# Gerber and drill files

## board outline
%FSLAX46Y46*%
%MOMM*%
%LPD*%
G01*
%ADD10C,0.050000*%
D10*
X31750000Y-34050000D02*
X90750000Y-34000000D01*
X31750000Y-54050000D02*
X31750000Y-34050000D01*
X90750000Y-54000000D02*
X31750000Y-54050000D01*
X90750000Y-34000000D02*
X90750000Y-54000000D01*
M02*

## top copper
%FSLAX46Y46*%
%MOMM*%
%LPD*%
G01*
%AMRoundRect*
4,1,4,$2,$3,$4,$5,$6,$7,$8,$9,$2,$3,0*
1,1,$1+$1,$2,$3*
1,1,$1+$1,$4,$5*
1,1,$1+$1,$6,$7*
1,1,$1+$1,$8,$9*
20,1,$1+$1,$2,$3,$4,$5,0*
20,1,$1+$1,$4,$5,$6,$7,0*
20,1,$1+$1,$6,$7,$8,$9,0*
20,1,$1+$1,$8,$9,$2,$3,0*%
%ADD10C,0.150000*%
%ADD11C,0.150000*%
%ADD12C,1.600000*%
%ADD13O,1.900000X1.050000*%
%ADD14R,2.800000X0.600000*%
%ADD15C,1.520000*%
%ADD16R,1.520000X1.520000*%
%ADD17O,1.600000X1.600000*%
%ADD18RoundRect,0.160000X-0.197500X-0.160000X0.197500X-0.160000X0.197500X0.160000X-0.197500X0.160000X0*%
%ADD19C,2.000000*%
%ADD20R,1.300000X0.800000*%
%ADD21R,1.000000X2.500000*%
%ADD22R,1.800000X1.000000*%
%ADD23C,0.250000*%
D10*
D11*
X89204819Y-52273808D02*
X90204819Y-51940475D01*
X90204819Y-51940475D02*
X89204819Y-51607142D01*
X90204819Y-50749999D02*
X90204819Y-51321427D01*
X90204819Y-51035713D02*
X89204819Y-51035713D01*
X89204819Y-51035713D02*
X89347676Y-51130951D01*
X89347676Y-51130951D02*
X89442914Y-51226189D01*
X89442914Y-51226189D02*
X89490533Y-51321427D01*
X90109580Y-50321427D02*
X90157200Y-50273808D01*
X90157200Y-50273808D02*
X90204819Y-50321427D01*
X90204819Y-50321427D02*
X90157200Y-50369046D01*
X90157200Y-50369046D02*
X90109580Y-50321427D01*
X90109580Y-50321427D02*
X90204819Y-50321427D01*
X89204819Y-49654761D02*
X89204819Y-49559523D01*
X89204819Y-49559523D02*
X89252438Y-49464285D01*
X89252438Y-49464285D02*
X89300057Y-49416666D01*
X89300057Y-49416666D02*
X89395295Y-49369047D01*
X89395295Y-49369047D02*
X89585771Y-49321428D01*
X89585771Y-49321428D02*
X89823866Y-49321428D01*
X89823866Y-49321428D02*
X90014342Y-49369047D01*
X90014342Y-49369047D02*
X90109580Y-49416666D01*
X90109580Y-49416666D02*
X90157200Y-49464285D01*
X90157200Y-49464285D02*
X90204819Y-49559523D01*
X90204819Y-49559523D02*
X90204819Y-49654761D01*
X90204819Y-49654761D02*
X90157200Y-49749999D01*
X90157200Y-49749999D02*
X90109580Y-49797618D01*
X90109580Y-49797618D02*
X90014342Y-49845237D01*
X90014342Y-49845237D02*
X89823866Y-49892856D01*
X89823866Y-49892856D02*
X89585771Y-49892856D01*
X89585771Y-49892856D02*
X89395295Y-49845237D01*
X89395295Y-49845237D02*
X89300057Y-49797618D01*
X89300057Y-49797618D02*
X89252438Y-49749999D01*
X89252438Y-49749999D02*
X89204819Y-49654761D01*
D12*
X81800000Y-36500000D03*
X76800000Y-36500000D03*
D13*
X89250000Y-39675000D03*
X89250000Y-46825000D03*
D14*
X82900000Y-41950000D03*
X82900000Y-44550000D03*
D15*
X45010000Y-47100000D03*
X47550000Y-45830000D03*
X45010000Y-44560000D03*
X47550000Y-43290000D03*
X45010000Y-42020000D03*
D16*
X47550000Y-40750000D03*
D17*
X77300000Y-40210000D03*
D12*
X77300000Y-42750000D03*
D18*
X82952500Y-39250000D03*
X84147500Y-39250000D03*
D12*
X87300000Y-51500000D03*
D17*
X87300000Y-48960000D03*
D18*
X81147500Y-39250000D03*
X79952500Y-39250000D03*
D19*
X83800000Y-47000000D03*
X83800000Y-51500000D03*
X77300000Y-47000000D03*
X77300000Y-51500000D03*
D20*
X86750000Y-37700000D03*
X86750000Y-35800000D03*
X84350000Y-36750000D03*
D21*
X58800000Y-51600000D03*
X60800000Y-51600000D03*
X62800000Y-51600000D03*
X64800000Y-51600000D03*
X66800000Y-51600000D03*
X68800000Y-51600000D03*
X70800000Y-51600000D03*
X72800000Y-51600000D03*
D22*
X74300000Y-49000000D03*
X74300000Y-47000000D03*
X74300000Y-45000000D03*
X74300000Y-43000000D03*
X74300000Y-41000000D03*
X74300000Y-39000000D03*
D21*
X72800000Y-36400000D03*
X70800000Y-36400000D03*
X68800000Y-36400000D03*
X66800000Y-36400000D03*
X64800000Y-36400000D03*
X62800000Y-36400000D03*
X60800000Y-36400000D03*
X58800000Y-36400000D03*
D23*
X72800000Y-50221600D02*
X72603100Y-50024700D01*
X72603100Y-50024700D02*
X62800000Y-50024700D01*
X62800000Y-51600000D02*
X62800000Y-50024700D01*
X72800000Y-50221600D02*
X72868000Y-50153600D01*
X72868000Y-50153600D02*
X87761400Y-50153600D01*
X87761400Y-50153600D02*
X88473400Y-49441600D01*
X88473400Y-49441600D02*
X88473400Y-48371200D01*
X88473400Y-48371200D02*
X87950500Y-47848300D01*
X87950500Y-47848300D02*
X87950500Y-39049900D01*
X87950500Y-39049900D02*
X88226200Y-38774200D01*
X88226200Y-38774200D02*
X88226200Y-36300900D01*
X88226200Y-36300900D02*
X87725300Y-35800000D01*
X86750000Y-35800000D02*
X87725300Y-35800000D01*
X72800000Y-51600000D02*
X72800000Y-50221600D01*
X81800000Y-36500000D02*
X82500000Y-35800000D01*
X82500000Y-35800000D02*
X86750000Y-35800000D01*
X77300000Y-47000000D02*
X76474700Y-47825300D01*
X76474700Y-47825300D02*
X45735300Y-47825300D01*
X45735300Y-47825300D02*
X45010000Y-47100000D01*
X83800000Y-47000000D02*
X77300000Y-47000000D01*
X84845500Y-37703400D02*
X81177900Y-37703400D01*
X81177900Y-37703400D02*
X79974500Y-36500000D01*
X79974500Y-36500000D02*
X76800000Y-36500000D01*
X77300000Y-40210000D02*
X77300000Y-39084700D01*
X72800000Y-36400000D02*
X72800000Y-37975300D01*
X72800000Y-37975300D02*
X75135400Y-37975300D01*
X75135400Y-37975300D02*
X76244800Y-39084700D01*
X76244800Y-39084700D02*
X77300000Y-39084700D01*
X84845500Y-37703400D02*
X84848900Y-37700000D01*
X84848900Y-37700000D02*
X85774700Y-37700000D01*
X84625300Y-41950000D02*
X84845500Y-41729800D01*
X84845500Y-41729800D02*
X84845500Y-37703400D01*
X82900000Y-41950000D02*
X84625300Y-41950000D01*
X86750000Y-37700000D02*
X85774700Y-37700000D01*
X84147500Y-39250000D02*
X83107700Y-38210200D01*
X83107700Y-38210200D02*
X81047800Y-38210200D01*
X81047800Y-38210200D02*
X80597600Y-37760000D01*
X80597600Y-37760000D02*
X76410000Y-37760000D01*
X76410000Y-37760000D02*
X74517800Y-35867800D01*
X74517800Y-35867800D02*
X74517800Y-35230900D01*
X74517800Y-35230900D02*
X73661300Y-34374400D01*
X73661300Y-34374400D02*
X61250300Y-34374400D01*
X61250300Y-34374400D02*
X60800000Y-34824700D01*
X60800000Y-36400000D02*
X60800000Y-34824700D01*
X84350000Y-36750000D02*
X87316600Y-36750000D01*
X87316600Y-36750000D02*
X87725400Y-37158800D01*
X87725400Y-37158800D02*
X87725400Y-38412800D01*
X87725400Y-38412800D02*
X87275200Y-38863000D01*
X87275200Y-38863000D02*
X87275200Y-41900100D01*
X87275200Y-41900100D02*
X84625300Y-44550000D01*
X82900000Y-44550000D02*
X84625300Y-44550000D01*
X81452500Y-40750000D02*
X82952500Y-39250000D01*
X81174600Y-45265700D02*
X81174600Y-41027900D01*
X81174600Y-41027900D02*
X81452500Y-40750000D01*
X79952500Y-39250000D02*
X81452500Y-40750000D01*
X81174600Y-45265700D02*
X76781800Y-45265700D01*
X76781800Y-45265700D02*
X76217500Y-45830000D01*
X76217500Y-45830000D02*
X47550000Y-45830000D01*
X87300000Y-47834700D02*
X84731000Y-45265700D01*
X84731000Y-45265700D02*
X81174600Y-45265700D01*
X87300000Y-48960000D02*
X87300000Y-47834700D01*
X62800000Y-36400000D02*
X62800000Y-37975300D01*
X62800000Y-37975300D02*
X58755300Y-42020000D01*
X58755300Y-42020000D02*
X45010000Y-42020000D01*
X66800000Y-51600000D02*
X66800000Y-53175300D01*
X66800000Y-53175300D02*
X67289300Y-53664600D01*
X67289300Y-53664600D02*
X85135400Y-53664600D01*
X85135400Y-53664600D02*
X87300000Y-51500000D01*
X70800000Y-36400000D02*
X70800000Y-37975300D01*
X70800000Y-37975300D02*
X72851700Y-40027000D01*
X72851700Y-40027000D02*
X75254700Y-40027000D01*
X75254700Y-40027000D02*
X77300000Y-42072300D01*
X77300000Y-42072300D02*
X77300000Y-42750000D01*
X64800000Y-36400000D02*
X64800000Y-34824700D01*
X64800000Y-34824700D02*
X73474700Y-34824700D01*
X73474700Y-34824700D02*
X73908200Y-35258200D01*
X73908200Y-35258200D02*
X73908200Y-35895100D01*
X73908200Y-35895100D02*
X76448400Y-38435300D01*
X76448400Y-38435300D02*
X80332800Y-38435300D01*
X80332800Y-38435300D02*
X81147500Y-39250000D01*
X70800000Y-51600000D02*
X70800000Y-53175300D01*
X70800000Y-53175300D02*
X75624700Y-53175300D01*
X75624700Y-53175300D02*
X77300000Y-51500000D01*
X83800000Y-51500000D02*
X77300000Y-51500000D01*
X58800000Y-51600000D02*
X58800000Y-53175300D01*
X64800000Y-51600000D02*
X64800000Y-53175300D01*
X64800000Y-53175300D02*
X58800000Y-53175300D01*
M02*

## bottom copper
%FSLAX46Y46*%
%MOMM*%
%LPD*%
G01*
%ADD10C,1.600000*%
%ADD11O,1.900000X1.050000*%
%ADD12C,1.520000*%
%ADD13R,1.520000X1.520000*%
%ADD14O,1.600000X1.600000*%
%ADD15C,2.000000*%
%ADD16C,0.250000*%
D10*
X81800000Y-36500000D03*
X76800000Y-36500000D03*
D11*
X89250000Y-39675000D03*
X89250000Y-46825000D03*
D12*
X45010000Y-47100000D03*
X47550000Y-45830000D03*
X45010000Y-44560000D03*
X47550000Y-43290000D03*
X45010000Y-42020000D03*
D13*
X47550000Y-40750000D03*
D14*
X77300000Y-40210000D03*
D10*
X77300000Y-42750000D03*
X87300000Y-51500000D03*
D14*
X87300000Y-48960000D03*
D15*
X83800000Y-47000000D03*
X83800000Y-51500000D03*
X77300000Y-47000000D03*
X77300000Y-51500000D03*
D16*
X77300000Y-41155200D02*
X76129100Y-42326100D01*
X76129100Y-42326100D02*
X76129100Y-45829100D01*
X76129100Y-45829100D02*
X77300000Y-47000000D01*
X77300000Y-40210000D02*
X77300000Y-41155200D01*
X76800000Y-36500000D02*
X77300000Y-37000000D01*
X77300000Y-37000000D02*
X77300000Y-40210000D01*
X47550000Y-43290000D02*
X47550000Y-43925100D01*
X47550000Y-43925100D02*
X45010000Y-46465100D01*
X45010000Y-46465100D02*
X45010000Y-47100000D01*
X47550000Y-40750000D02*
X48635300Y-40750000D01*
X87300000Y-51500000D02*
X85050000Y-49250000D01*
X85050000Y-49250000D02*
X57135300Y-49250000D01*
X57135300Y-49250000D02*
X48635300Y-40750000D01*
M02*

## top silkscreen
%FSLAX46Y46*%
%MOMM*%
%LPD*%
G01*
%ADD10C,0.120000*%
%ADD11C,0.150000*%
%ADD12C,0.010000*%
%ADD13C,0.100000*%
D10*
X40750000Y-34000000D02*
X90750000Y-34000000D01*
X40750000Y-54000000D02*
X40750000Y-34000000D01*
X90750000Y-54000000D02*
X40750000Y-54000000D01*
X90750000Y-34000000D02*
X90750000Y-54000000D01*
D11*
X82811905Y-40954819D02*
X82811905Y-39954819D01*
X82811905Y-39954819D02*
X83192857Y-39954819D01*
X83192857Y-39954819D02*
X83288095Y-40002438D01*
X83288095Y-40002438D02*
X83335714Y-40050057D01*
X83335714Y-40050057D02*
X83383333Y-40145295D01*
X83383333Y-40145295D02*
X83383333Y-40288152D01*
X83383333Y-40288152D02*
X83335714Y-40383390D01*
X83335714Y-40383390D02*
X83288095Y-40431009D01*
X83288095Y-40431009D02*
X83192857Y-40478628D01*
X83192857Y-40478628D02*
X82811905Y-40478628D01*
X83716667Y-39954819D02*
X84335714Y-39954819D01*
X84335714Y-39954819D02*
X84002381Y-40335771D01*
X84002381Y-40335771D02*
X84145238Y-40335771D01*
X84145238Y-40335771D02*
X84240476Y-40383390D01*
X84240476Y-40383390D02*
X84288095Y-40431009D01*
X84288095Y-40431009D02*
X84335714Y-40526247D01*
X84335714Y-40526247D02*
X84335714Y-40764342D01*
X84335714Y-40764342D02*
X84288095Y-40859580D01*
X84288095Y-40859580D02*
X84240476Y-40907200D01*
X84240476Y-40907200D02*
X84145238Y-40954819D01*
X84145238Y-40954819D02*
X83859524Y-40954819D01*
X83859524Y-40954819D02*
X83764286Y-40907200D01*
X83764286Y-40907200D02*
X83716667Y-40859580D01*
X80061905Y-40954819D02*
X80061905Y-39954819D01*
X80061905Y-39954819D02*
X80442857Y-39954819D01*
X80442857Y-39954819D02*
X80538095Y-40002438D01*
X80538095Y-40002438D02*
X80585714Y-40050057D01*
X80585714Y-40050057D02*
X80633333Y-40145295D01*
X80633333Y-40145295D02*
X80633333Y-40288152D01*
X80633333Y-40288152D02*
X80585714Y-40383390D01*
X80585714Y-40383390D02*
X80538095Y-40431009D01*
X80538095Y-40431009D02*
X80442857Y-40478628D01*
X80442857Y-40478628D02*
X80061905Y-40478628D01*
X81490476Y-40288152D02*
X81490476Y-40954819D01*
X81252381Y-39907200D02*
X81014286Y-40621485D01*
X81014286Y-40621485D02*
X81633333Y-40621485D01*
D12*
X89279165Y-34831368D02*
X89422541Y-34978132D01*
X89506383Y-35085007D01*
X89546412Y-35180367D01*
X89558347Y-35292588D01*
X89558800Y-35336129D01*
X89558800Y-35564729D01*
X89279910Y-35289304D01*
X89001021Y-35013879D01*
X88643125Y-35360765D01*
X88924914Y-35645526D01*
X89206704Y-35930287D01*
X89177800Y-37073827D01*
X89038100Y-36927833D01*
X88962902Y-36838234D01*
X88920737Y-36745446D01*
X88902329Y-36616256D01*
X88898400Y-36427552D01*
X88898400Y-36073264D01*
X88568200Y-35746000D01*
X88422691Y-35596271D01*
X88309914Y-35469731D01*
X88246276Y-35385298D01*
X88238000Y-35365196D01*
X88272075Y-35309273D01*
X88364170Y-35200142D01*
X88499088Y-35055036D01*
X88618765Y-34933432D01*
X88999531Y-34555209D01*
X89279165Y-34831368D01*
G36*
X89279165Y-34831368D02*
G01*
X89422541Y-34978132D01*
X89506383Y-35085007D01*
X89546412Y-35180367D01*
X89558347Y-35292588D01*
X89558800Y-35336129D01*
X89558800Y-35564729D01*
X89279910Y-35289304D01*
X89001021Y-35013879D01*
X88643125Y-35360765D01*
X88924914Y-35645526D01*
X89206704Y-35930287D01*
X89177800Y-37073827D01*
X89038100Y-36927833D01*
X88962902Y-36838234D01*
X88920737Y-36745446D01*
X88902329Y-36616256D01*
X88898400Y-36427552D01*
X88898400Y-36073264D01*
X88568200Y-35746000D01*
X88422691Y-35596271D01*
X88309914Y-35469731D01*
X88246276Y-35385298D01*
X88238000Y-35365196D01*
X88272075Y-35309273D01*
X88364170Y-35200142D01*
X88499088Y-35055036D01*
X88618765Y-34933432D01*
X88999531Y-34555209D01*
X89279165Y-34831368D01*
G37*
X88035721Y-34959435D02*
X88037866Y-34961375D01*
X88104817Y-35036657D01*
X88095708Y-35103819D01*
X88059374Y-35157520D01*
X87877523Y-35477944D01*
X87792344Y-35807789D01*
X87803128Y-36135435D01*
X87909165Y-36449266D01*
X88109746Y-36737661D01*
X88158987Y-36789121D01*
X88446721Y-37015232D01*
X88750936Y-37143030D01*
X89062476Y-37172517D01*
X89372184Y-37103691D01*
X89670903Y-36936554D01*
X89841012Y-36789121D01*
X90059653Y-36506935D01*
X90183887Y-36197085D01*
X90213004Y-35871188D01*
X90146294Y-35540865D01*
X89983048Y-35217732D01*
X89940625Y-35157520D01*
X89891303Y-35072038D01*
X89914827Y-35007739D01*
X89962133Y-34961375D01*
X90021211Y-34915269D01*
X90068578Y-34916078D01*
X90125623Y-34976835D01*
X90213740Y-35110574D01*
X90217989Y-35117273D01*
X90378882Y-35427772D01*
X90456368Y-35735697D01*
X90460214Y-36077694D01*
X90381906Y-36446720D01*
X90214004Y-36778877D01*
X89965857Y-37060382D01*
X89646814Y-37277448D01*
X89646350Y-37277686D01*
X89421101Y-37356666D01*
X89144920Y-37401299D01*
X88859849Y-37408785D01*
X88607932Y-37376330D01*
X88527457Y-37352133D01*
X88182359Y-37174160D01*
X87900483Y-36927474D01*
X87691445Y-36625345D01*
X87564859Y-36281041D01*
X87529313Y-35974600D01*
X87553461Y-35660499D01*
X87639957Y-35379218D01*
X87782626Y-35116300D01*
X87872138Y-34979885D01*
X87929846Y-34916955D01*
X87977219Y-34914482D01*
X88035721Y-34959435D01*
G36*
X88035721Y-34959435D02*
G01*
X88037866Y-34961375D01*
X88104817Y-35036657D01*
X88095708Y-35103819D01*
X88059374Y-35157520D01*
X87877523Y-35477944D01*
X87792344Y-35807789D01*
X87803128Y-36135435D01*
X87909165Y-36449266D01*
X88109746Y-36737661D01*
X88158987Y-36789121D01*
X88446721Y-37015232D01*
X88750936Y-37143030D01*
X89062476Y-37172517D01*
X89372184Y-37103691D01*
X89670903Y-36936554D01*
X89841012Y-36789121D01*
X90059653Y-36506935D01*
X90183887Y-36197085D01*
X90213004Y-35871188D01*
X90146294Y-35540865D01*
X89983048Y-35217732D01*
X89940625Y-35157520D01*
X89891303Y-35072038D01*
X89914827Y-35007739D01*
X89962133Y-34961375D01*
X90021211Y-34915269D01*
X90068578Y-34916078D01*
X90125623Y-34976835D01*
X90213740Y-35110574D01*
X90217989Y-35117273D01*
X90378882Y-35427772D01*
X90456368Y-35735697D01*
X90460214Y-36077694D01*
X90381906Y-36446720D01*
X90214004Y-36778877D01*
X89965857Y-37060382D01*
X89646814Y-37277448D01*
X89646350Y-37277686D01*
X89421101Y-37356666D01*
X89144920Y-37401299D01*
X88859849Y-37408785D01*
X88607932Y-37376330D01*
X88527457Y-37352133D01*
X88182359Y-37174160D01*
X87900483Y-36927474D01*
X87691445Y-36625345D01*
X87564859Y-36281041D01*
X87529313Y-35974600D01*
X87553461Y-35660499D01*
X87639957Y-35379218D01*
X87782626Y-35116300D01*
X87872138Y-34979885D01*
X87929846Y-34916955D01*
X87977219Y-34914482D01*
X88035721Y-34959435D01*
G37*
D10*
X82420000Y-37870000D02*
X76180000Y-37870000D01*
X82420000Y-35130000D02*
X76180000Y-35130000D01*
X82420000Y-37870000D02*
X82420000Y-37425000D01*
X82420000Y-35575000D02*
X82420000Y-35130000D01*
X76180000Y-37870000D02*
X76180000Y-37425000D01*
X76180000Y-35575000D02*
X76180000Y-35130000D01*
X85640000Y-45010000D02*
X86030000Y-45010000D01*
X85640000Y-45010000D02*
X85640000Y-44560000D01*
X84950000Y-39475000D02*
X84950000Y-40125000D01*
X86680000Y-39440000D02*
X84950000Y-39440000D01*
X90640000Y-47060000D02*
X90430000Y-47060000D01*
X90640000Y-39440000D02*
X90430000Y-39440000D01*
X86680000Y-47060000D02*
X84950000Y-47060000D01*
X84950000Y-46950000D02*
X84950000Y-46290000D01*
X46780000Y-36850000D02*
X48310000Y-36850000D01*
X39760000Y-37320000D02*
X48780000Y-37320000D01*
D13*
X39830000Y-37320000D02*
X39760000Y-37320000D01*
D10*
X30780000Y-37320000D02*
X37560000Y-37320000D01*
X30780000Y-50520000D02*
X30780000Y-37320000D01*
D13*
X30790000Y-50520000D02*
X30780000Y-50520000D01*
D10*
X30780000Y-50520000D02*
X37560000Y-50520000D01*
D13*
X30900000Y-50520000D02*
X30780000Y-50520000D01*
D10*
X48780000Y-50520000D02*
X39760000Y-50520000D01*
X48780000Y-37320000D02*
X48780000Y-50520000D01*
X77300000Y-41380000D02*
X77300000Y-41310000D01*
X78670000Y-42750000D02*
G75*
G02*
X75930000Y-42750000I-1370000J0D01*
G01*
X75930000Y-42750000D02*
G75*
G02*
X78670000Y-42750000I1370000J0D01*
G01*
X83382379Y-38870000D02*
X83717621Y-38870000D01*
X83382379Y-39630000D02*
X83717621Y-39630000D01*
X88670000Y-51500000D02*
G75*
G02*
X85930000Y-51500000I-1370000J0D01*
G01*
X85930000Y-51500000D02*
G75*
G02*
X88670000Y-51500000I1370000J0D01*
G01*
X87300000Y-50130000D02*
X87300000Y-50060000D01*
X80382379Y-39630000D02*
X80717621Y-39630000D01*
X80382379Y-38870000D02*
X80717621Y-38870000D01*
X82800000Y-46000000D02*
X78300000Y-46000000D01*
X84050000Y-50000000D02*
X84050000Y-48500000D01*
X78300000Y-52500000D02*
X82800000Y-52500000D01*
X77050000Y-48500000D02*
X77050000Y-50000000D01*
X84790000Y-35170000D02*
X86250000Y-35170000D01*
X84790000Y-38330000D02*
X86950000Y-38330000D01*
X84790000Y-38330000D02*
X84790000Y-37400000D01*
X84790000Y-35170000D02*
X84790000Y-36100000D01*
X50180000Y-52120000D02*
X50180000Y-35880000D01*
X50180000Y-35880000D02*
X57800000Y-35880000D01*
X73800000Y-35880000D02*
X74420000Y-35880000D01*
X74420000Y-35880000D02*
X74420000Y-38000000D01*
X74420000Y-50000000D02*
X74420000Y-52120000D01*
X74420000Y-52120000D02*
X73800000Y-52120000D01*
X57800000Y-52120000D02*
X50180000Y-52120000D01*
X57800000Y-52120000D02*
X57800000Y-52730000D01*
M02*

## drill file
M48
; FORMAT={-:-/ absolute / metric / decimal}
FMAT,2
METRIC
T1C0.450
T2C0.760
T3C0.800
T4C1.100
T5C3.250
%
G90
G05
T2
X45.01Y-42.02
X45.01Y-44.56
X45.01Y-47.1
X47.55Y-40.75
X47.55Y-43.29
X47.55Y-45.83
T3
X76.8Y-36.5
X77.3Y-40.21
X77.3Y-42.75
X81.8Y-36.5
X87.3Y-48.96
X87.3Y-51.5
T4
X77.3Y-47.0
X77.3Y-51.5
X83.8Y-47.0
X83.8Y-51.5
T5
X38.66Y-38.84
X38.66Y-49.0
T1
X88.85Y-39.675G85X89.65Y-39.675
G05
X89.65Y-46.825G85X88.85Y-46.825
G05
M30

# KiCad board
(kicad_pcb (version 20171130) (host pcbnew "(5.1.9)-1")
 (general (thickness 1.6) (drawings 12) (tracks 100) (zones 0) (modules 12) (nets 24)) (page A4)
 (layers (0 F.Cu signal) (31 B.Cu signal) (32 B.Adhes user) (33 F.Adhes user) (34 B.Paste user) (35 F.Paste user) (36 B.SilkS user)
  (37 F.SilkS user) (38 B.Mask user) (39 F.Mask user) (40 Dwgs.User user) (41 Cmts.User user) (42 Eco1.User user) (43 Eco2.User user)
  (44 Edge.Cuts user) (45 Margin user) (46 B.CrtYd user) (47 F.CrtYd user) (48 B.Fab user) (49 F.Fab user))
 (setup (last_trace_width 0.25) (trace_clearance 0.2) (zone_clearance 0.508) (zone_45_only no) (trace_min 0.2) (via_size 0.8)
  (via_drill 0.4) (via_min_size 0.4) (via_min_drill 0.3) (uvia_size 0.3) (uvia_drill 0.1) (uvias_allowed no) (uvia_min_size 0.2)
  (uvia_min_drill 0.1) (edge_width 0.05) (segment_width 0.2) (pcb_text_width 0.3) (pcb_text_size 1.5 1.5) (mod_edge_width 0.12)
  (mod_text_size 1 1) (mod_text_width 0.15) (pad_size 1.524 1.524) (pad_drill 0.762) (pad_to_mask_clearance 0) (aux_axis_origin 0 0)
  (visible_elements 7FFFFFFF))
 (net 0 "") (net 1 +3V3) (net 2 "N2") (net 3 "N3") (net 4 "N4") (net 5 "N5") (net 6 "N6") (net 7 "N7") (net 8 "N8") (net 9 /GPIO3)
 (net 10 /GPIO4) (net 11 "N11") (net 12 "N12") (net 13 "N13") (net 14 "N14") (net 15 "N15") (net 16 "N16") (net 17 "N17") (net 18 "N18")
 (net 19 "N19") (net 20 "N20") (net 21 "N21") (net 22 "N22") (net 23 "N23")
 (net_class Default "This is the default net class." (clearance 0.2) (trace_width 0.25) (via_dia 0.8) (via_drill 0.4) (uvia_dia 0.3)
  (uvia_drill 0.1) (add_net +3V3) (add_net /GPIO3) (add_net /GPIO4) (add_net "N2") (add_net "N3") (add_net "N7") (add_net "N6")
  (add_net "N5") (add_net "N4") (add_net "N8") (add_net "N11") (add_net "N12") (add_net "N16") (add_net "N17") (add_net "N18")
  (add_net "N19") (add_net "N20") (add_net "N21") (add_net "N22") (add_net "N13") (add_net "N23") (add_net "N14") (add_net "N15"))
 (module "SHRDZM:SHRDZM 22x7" (layer B.Cu) (at 63 43.25 180)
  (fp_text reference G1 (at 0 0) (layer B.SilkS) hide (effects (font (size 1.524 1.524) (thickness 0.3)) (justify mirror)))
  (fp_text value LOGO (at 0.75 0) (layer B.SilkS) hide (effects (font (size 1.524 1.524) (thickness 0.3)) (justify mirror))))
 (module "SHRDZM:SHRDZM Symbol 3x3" (layer F.Cu) (at 89 36)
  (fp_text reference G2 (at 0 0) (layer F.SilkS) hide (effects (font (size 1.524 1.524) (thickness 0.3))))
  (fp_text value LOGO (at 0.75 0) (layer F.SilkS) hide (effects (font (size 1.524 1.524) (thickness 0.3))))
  (fp_poly
   (pts (xy 0.279165 -1.168632) (xy 0.422541 -1.021868) (xy 0.506383 -0.914993) (xy 0.546412 -0.819633) (xy 0.558347 -0.707412)
    (xy 0.5588 -0.663871) (xy 0.5588 -0.435271) (xy 0.27991 -0.710696) (xy 0.001021 -0.986121) (xy -0.356875 -0.639235)
    (xy -0.075086 -0.354474) (xy 0.206704 -0.069713) (xy 0.1778 1.073827) (xy 0.0381 0.927833) (xy -0.037098 0.838234)
    (xy -0.079263 0.745446) (xy -0.097671 0.616256) (xy -0.1016 0.427552) (xy -0.1016 0.073264) (xy -0.4318 -0.254) (xy -0.577309 -0.403729)
    (xy -0.690086 -0.530269) (xy -0.753724 -0.614702) (xy -0.762 -0.634804) (xy -0.727925 -0.690727) (xy -0.63583 -0.799858)
    (xy -0.500912 -0.944964) (xy -0.381235 -1.066568) (xy -0.000469 -1.444791) (xy 0.279165 -1.168632))
   (layer F.SilkS) (width 0.01))
  (fp_poly
   (pts (xy -0.964279 -1.040565) (xy -0.962134 -1.038625) (xy -0.895183 -0.963343) (xy -0.904292 -0.896181) (xy -0.940626 -0.84248)
    (xy -1.122477 -0.522056) (xy -1.207656 -0.192211) (xy -1.196872 0.135435) (xy -1.090835 0.449266) (xy -0.890254 0.737661)
    (xy -0.841013 0.789121) (xy -0.553279 1.015232) (xy -0.249064 1.14303) (xy 0.062476 1.172517) (xy 0.372184 1.103691)
    (xy 0.670903 0.936554) (xy 0.841012 0.789121) (xy 1.059653 0.506935) (xy 1.183887 0.197085) (xy 1.213004 -0.128812)
    (xy 1.146294 -0.459135) (xy 0.983048 -0.782268) (xy 0.940625 -0.84248) (xy 0.891303 -0.927962) (xy 0.914827 -0.992261)
    (xy 0.962133 -1.038625) (xy 1.021211 -1.084731) (xy 1.068578 -1.083922) (xy 1.125623 -1.023165) (xy 1.21374 -0.889426)
    (xy 1.217989 -0.882727) (xy 1.378882 -0.572228) (xy 1.456368 -0.264303) (xy 1.460214 0.077694) (xy 1.381906 0.44672)
    (xy 1.214004 0.778877) (xy 0.965857 1.060382) (xy 0.646814 1.277448) (xy 0.64635 1.277686) (xy 0.421101 1.356666) (xy 0.14492 1.401299)
    (xy -0.140151 1.408785) (xy -0.392068 1.37633) (xy -0.472543 1.352133) (xy -0.817641 1.17416) (xy -1.099517 0.927474)
    (xy -1.308555 0.625345) (xy -1.435141 0.281041) (xy -1.470687 -0.0254) (xy -1.446539 -0.339501) (xy -1.360043 -0.620782)
    (xy -1.217374 -0.8837) (xy -1.127862 -1.020115) (xy -1.070154 -1.083045) (xy -1.022781 -1.085518) (xy -0.964279 -1.040565))
   (layer F.SilkS) (width 0.01)))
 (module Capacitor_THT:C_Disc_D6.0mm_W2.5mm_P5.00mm (layer F.Cu) (at 81.8 36.5 180)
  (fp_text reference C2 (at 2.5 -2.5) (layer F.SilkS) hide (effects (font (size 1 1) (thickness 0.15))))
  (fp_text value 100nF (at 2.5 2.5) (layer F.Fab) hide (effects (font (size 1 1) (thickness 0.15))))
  (fp_line (start -0.62 -1.37) (end 5.62 -1.37) (layer F.SilkS) (width 0.12))
  (fp_line (start -0.62 1.37) (end 5.62 1.37) (layer F.SilkS) (width 0.12))
  (fp_line (start -0.62 -1.37) (end -0.62 -0.925) (layer F.SilkS) (width 0.12))
  (fp_line (start -0.62 0.925) (end -0.62 1.37) (layer F.SilkS) (width 0.12))
  (fp_line (start 5.62 -1.37) (end 5.62 -0.925) (layer F.SilkS) (width 0.12))
  (fp_line (start 5.62 0.925) (end 5.62 1.37) (layer F.SilkS) (width 0.12))
  (pad 1 thru_hole circle (at 0 0 180) (size 1.6 1.6) (drill 0.8) (layers *.Cu *.Mask) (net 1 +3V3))
  (pad 2 thru_hole circle (at 5 0 180) (size 1.6 1.6) (drill 0.8) (layers *.Cu *.Mask) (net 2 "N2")))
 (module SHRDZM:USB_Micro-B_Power (layer F.Cu) (at 88.05 43.25 90)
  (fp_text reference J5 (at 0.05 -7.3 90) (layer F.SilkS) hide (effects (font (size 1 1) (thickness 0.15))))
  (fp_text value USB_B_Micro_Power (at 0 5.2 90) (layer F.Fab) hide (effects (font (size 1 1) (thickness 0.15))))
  (fp_line (start -1.76 -2.41) (end -1.76 -2.02) (layer F.SilkS) (width 0.12))
  (fp_line (start -1.76 -2.41) (end -1.31 -2.41) (layer F.SilkS) (width 0.12))
  (fp_line (start 3.775 -3.1) (end 3.125 -3.1) (layer F.SilkS) (width 0.12))
  (fp_line (start 3.81 -1.37) (end 3.81 -3.1) (layer F.SilkS) (width 0.12))
  (fp_line (start -3.81 2.59) (end -3.81 2.38) (layer F.SilkS) (width 0.12))
  (fp_line (start 3.81 2.59) (end 3.81 2.38) (layer F.SilkS) (width 0.12))
  (fp_line (start -3.81 -1.37) (end -3.81 -3.1) (layer F.SilkS) (width 0.12))
  (fp_line (start -3.7 -3.1) (end -3.04 -3.1) (layer F.SilkS) (width 0.12))
  (pad "" thru_hole oval (at 3.575 1.2 90) (size 1.05 1.9) (drill oval 0.45 1.25) (layers *.Cu *.Mask))
  (pad "" thru_hole oval (at -3.575 1.2 270) (size 1.05 1.9) (drill oval 0.45 1.25) (layers *.Cu *.Mask))
  (pad 5 smd rect (at 1.3 -5.15 90) (size 0.6 2.8) (layers F.Cu F.Paste F.Mask) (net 2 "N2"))
  (pad 1 smd rect (at -1.3 -5.15 90) (size 0.6 2.8) (layers F.Cu F.Paste F.Mask) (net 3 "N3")))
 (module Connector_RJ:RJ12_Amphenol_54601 (layer F.Cu) (at 47.55 40.75 270)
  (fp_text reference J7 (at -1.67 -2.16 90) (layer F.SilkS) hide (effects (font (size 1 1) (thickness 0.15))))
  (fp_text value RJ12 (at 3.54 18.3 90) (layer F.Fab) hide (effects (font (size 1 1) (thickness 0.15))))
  (fp_line (start -3.9 0.77) (end -3.9 -0.76) (layer F.SilkS) (width 0.12))
  (fp_line (start -3.43 7.79) (end -3.43 -1.23) (layer F.SilkS) (width 0.12))
  (fp_line (start -3.43 7.72) (end -3.43 7.79) (layer F.SilkS) (width 0.1))
  (fp_line (start -3.43 16.77) (end -3.43 9.99) (layer F.SilkS) (width 0.12))
  (fp_line (start 9.77 16.77) (end -3.43 16.77) (layer F.SilkS) (width 0.12))
  (fp_line (start 9.77 16.76) (end 9.77 16.77) (layer F.SilkS) (width 0.1))
  (fp_line (start 9.77 16.77) (end 9.77 9.99) (layer F.SilkS) (width 0.12))
  (fp_line (start 9.77 16.65) (end 9.77 16.77) (layer F.SilkS) (width 0.1))
  (fp_line (start 9.77 -1.23) (end 9.77 7.79) (layer F.SilkS) (width 0.12))
  (fp_line (start -3.43 -1.23) (end 9.77 -1.23) (layer F.SilkS) (width 0.12))
  (pad "" np_thru_hole circle (at 8.25 8.89 270) (size 3.25 3.25) (drill 3.25) (layers *.Cu *.Mask))
  (pad 6 thru_hole circle (at 6.35 2.54 270) (size 1.52 1.52) (drill 0.76) (layers *.Cu *.Mask) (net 2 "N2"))
  (pad 5 thru_hole circle (at 5.08 0 270) (size 1.52 1.52) (drill 0.76) (layers *.Cu *.Mask) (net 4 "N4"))
  (pad 4 thru_hole circle (at 3.81 2.54 270) (size 1.52 1.52) (drill 0.76) (layers *.Cu *.Mask) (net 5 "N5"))
  (pad 3 thru_hole circle (at 2.54 0 270) (size 1.52 1.52) (drill 0.76) (layers *.Cu *.Mask) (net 2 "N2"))
  (pad 2 thru_hole circle (at 1.27 2.54 270) (size 1.52 1.52) (drill 0.76) (layers *.Cu *.Mask) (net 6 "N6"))
  (pad "" np_thru_hole circle (at -1.91 8.89 270) (size 3.25 3.25) (drill 3.25) (layers *.Cu *.Mask))
  (pad 1 thru_hole rect (at 0 0 270) (size 1.52 1.52) (drill 0.76) (layers *.Cu *.Mask) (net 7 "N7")))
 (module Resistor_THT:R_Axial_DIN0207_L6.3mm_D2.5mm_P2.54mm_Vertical (layer F.Cu) (at 77.3 42.75 90)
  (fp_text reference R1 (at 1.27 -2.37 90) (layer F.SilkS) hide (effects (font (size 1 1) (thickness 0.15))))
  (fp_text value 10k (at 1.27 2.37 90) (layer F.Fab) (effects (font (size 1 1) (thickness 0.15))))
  (fp_line (start 1.37 0) (end 1.44 0) (layer F.SilkS) (width 0.12))
  (fp_circle (center 0 0) (end 1.37 0) (layer F.SilkS) (width 0.12))
  (pad 2 thru_hole oval (at 2.54 0 90) (size 1.6 1.6) (drill 0.8) (layers *.Cu *.Mask) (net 2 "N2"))
  (pad 1 thru_hole circle (at 0 0 90) (size 1.6 1.6) (drill 0.8) (layers *.Cu *.Mask) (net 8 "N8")))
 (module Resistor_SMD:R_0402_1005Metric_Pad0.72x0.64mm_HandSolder (layer F.Cu) (at 83.55 39.25)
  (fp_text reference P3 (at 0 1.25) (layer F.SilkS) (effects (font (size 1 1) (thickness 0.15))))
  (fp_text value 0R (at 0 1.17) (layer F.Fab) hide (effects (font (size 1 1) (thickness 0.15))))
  (fp_line (start -0.167621 -0.38) (end 0.167621 -0.38) (layer F.SilkS) (width 0.12))
  (fp_line (start -0.167621 0.38) (end 0.167621 0.38) (layer F.SilkS) (width 0.12))
  (pad 1 smd roundrect (at -0.5975 0) (size 0.715 0.64) (layers F.Cu F.Paste F.Mask) (roundrect_rratio 0.25) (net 4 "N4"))
  (pad 2 smd roundrect (at 0.5975 0) (size 0.715 0.64) (layers F.Cu F.Paste F.Mask) (roundrect_rratio 0.25) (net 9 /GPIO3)))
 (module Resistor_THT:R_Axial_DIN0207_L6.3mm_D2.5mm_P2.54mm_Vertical (layer F.Cu) (at 87.3 51.5 90)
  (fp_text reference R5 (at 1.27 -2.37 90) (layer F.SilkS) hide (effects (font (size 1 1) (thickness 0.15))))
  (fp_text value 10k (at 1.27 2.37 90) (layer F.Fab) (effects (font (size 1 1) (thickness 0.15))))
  (fp_circle (center 0 0) (end 1.37 0) (layer F.SilkS) (width 0.12))
  (fp_line (start 1.37 0) (end 1.44 0) (layer F.SilkS) (width 0.12))
  (pad 1 thru_hole circle (at 0 0 90) (size 1.6 1.6) (drill 0.8) (layers *.Cu *.Mask) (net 7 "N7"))
  (pad 2 thru_hole oval (at 2.54 0 90) (size 1.6 1.6) (drill 0.8) (layers *.Cu *.Mask) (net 4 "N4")))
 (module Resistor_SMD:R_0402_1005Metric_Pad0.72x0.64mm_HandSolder (layer F.Cu) (at 80.55 39.25)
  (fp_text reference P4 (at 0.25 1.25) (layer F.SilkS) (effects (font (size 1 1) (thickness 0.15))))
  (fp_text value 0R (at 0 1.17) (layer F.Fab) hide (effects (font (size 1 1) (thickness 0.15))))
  (fp_line (start -0.167621 0.38) (end 0.167621 0.38) (layer F.SilkS) (width 0.12))
  (fp_line (start -0.167621 -0.38) (end 0.167621 -0.38) (layer F.SilkS) (width 0.12))
  (pad 2 smd roundrect (at 0.5975 0) (size 0.715 0.64) (layers F.Cu F.Paste F.Mask) (roundrect_rratio 0.25) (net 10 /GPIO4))
  (pad 1 smd roundrect (at -0.5975 0) (size 0.715 0.64) (layers F.Cu F.Paste F.Mask) (roundrect_rratio 0.25) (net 4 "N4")))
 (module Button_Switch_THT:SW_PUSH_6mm (layer F.Cu) (at 83.8 51.5 180)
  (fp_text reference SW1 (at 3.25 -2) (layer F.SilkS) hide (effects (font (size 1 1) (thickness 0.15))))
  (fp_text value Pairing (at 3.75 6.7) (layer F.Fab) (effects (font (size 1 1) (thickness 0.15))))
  (fp_line (start 1 5.5) (end 5.5 5.5) (layer F.SilkS) (width 0.12))
  (fp_line (start -0.25 1.5) (end -0.25 3) (layer F.SilkS) (width 0.12))
  (fp_line (start 5.5 -1) (end 1 -1) (layer F.SilkS) (width 0.12))
  (fp_line (start 6.75 3) (end 6.75 1.5) (layer F.SilkS) (width 0.12))
  (pad 2 thru_hole circle (at 0 4.5 270) (size 2 2) (drill 1.1) (layers *.Cu *.Mask) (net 2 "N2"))
  (pad 1 thru_hole circle (at 0 0 270) (size 2 2) (drill 1.1) (layers *.Cu *.Mask) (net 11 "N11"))
  (pad 2 thru_hole circle (at 6.5 4.5 270) (size 2 2) (drill 1.1) (layers *.Cu *.Mask) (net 2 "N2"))
  (pad 1 thru_hole circle (at 6.5 0 270) (size 2 2) (drill 1.1) (layers *.Cu *.Mask) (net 11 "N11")))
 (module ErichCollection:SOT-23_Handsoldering (layer F.Cu) (at 85.55 36.75 180)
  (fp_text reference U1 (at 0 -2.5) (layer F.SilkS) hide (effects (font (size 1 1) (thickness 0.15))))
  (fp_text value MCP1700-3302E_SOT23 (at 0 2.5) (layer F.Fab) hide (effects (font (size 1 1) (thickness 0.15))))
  (fp_line (start 0.76 1.58) (end -0.7 1.58) (layer F.SilkS) (width 0.12))
  (fp_line (start 0.76 -1.58) (end -1.4 -1.58) (layer F.SilkS) (width 0.12))
  (fp_line (start 0.76 -1.58) (end 0.76 -0.65) (layer F.SilkS) (width 0.12))
  (fp_line (start 0.76 1.58) (end 0.76 0.65) (layer F.SilkS) (width 0.12))
  (pad 1 smd rect (at -1.2 -0.95 180) (size 1.3 0.8) (layers F.Cu F.Paste F.Mask) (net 2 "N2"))
  (pad 2 smd rect (at -1.2 0.95 180) (size 1.3 0.8) (layers F.Cu F.Paste F.Mask) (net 1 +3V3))
  (pad 3 smd rect (at 1.2 0 180) (size 1.3 0.8) (layers F.Cu F.Paste F.Mask) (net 3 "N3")))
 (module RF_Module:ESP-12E (layer F.Cu) (at 62.3 44 90)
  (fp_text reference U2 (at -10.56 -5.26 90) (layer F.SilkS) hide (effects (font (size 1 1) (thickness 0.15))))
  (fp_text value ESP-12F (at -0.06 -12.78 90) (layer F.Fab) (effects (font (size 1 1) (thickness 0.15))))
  (fp_line (start -8.12 -12.12) (end 8.12 -12.12) (layer F.SilkS) (width 0.12))
  (fp_line (start 8.12 -12.12) (end 8.12 -4.5) (layer F.SilkS) (width 0.12))
  (fp_line (start 8.12 11.5) (end 8.12 12.12) (layer F.SilkS) (width 0.12))
  (fp_line (start 8.12 12.12) (end 6 12.12) (layer F.SilkS) (width 0.12))
  (fp_line (start -6 12.12) (end -8.12 12.12) (layer F.SilkS) (width 0.12))
  (fp_line (start -8.12 12.12) (end -8.12 11.5) (layer F.SilkS) (width 0.12))
  (fp_line (start -8.12 -4.5) (end -8.12 -12.12) (layer F.SilkS) (width 0.12))
  (fp_line (start -8.12 -4.5) (end -8.73 -4.5) (layer F.SilkS) (width 0.12))
  (pad 1 smd rect (at -7.6 -3.5 90) (size 2.5 1) (layers F.Cu F.Paste F.Mask) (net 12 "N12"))
  (pad 2 smd rect (at -7.6 -1.5 90) (size 2.5 1) (layers F.Cu F.Paste F.Mask) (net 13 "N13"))
  (pad 3 smd rect (at -7.6 0.5 90) (size 2.5 1) (layers F.Cu F.Paste F.Mask) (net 1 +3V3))
  (pad 4 smd rect (at -7.6 2.5 90) (size 2.5 1) (layers F.Cu F.Paste F.Mask) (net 12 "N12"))
  (pad 5 smd rect (at -7.6 4.5 90) (size 2.5 1) (layers F.Cu F.Paste F.Mask) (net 7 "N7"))
  (pad 6 smd rect (at -7.6 6.5 90) (size 2.5 1) (layers F.Cu F.Paste F.Mask) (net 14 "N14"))
  (pad 7 smd rect (at -7.6 8.5 90) (size 2.5 1) (layers F.Cu F.Paste F.Mask) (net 11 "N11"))
  (pad 8 smd rect (at -7.6 10.5 90) (size 2.5 1) (layers F.Cu F.Paste F.Mask) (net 1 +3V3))
  (pad 9 smd rect (at -5 12 90) (size 1 1.8) (layers F.Cu F.Paste F.Mask) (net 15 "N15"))
  (pad 10 smd rect (at -3 12 90) (size 1 1.8) (layers F.Cu F.Paste F.Mask) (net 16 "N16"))
  (pad 11 smd rect (at -1 12 90) (size 1 1.8) (layers F.Cu F.Paste F.Mask) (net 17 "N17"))
  (pad 12 smd rect (at 1 12 90) (size 1 1.8) (layers F.Cu F.Paste F.Mask) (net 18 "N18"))
  (pad 13 smd rect (at 3 12 90) (size 1 1.8) (layers F.Cu F.Paste F.Mask) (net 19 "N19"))
  (pad 14 smd rect (at 5 12 90) (size 1 1.8) (layers F.Cu F.Paste F.Mask) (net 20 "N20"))
  (pad 15 smd rect (at 7.6 10.5 90) (size 2.5 1) (layers F.Cu F.Paste F.Mask) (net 2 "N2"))
  (pad 16 smd rect (at 7.6 8.5 90) (size 2.5 1) (layers F.Cu F.Paste F.Mask) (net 8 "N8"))
  (pad 17 smd rect (at 7.6 6.5 90) (size 2.5 1) (layers F.Cu F.Paste F.Mask) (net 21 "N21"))
  (pad 18 smd rect (at 7.6 4.5 90) (size 2.5 1) (layers F.Cu F.Paste F.Mask) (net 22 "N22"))
  (pad 19 smd rect (at 7.6 2.5 90) (size 2.5 1) (layers F.Cu F.Paste F.Mask) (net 10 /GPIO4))
  (pad 20 smd rect (at 7.6 0.5 90) (size 2.5 1) (layers F.Cu F.Paste F.Mask) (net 6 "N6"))
  (pad 21 smd rect (at 7.6 -1.5 90) (size 2.5 1) (layers F.Cu F.Paste F.Mask) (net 9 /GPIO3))
  (pad 22 smd rect (at 7.6 -3.5 90) (size 2.5 1) (layers F.Cu F.Paste F.Mask) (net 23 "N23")))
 (gr_line (start 31.75 34.05) (end 90.75 34) (layer Edge.Cuts) (width 0.05))
 (gr_line (start 31.75 54.05) (end 31.75 34.05) (layer Edge.Cuts) (width 0.05))
 (gr_line (start 90.75 54) (end 31.75 54.05) (layer Edge.Cuts) (width 0.05))
 (gr_line (start 90.75 34) (end 90.75 54) (layer Edge.Cuts) (width 0.05))
 (gr_line (start 40.75 34) (end 90.75 34) (layer F.SilkS) (width 0.12))
 (gr_line (start 40.75 54) (end 40.75 34) (layer F.SilkS) (width 0.12))
 (gr_line (start 90.75 54) (end 40.75 54) (layer F.SilkS) (width 0.12))
 (gr_line (start 90.75 34) (end 90.75 54) (layer F.SilkS) (width 0.12))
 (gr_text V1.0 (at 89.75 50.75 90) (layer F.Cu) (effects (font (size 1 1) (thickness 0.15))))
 (segment (start 72.8 50.2216) (end 72.6031 50.0247) (width 0.25) (layer F.Cu) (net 1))
 (segment (start 72.6031 50.0247) (end 62.8 50.0247) (width 0.25) (layer F.Cu) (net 1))
 (segment (start 62.8 51.6) (end 62.8 50.0247) (width 0.25) (layer F.Cu) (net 1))
 (segment (start 72.8 50.2216) (end 72.868 50.1536) (width 0.25) (layer F.Cu) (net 1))
 (segment (start 72.868 50.1536) (end 87.7614 50.1536) (width 0.25) (layer F.Cu) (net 1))
 (segment (start 87.7614 50.1536) (end 88.4734 49.4416) (width 0.25) (layer F.Cu) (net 1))
 (segment (start 88.4734 49.4416) (end 88.4734 48.3712) (width 0.25) (layer F.Cu) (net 1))
 (segment (start 88.4734 48.3712) (end 87.9505 47.8483) (width 0.25) (layer F.Cu) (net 1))
 (segment (start 87.9505 47.8483) (end 87.9505 39.0499) (width 0.25) (layer F.Cu) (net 1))
 (segment (start 87.9505 39.0499) (end 88.2262 38.7742) (width 0.25) (layer F.Cu) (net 1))
 (segment (start 88.2262 38.7742) (end 88.2262 36.3009) (width 0.25) (layer F.Cu) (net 1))
 (segment (start 88.2262 36.3009) (end 87.7253 35.8) (width 0.25) (layer F.Cu) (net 1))
 (segment (start 86.75 35.8) (end 87.7253 35.8) (width 0.25) (layer F.Cu) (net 1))
 (segment (start 72.8 51.6) (end 72.8 50.2216) (width 0.25) (layer F.Cu) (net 1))
 (segment (start 81.8 36.5) (end 82.5 35.8) (width 0.25) (layer F.Cu) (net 1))
 (segment (start 82.5 35.8) (end 86.75 35.8) (width 0.25) (layer F.Cu) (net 1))
 (segment (start 77.3 47) (end 76.4747 47.8253) (width 0.25) (layer F.Cu) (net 2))
 (segment (start 76.4747 47.8253) (end 45.7353 47.8253) (width 0.25) (layer F.Cu) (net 2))
 (segment (start 45.7353 47.8253) (end 45.01 47.1) (width 0.25) (layer F.Cu) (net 2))
 (segment (start 83.8 47) (end 77.3 47) (width 0.25) (layer F.Cu) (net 2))
 (segment (start 84.8455 37.7034) (end 81.1779 37.7034) (width 0.25) (layer F.Cu) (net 2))
 (segment (start 81.1779 37.7034) (end 79.9745 36.5) (width 0.25) (layer F.Cu) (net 2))
 (segment (start 79.9745 36.5) (end 76.8 36.5) (width 0.25) (layer F.Cu) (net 2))
 (segment (start 77.3 40.21) (end 77.3 39.0847) (width 0.25) (layer F.Cu) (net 2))
 (segment (start 72.8 36.4) (end 72.8 37.9753) (width 0.25) (layer F.Cu) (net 2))
 (segment (start 72.8 37.9753) (end 75.1354 37.9753) (width 0.25) (layer F.Cu) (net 2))
 (segment (start 75.1354 37.9753) (end 76.2448 39.0847) (width 0.25) (layer F.Cu) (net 2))
 (segment (start 76.2448 39.0847) (end 77.3 39.0847) (width 0.25) (layer F.Cu) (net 2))
 (segment (start 77.3 41.1552) (end 76.1291 42.3261) (width 0.25) (layer B.Cu) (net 2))
 (segment (start 76.1291 42.3261) (end 76.1291 45.8291) (width 0.25) (layer B.Cu) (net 2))
 (segment (start 76.1291 45.8291) (end 77.3 47) (width 0.25) (layer B.Cu) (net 2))
 (segment (start 77.3 40.21) (end 77.3 41.1552) (width 0.25) (layer B.Cu) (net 2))
 (segment (start 76.8 36.5) (end 77.3 37) (width 0.25) (layer B.Cu) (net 2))
 (segment (start 77.3 37) (end 77.3 40.21) (width 0.25) (layer B.Cu) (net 2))
 (segment (start 84.8455 37.7034) (end 84.8489 37.7) (width 0.25) (layer F.Cu) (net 2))
 (segment (start 84.8489 37.7) (end 85.7747 37.7) (width 0.25) (layer F.Cu) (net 2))
 (segment (start 84.6253 41.95) (end 84.8455 41.7298) (width 0.25) (layer F.Cu) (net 2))
 (segment (start 84.8455 41.7298) (end 84.8455 37.7034) (width 0.25) (layer F.Cu) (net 2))
 (segment (start 82.9 41.95) (end 84.6253 41.95) (width 0.25) (layer F.Cu) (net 2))
 (segment (start 47.55 43.29) (end 47.55 43.9251) (width 0.25) (layer B.Cu) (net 2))
 (segment (start 47.55 43.9251) (end 45.01 46.4651) (width 0.25) (layer B.Cu) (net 2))
 (segment (start 45.01 46.4651) (end 45.01 47.1) (width 0.25) (layer B.Cu) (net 2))
 (segment (start 86.75 37.7) (end 85.7747 37.7) (width 0.25) (layer F.Cu) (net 2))
 (segment (start 84.1475 39.25) (end 83.1077 38.2102) (width 0.25) (layer F.Cu) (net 9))
 (segment (start 83.1077 38.2102) (end 81.0478 38.2102) (width 0.25) (layer F.Cu) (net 9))
 (segment (start 81.0478 38.2102) (end 80.5976 37.76) (width 0.25) (layer F.Cu) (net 9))
 (segment (start 80.5976 37.76) (end 76.41 37.76) (width 0.25) (layer F.Cu) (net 9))
 (segment (start 76.41 37.76) (end 74.5178 35.8678) (width 0.25) (layer F.Cu) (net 9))
 (segment (start 74.5178 35.8678) (end 74.5178 35.2309) (width 0.25) (layer F.Cu) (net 9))
 (segment (start 74.5178 35.2309) (end 73.6613 34.3744) (width 0.25) (layer F.Cu) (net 9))
 (segment (start 73.6613 34.3744) (end 61.2503 34.3744) (width 0.25) (layer F.Cu) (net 9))
 (segment (start 61.2503 34.3744) (end 60.8 34.8247) (width 0.25) (layer F.Cu) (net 9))
 (segment (start 60.8 36.4) (end 60.8 34.8247) (width 0.25) (layer F.Cu) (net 9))
 (segment (start 84.35 36.75) (end 87.3166 36.75) (width 0.25) (layer F.Cu) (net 3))
 (segment (start 87.3166 36.75) (end 87.7254 37.1588) (width 0.25) (layer F.Cu) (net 3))
 (segment (start 87.7254 37.1588) (end 87.7254 38.4128) (width 0.25) (layer F.Cu) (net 3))
 (segment (start 87.7254 38.4128) (end 87.2752 38.863) (width 0.25) (layer F.Cu) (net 3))
 (segment (start 87.2752 38.863) (end 87.2752 41.9001) (width 0.25) (layer F.Cu) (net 3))
 (segment (start 87.2752 41.9001) (end 84.6253 44.55) (width 0.25) (layer F.Cu) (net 3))
 (segment (start 82.9 44.55) (end 84.6253 44.55) (width 0.25) (layer F.Cu) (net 3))
 (segment (start 81.4525 40.75) (end 82.9525 39.25) (width 0.25) (layer F.Cu) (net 4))
 (segment (start 81.1746 45.2657) (end 81.1746 41.0279) (width 0.25) (layer F.Cu) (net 4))
 (segment (start 81.1746 41.0279) (end 81.4525 40.75) (width 0.25) (layer F.Cu) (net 4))
 (segment (start 79.9525 39.25) (end 81.4525 40.75) (width 0.25) (layer F.Cu) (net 4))
 (segment (start 81.1746 45.2657) (end 76.7818 45.2657) (width 0.25) (layer F.Cu) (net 4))
 (segment (start 76.7818 45.2657) (end 76.2175 45.83) (width 0.25) (layer F.Cu) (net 4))
 (segment (start 76.2175 45.83) (end 47.55 45.83) (width 0.25) (layer F.Cu) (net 4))
 (segment (start 87.3 47.8347) (end 84.731 45.2657) (width 0.25) (layer F.Cu) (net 4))
 (segment (start 84.731 45.2657) (end 81.1746 45.2657) (width 0.25) (layer F.Cu) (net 4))
 (segment (start 87.3 48.96) (end 87.3 47.8347) (width 0.25) (layer F.Cu) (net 4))
 (segment (start 62.8 36.4) (end 62.8 37.9753) (width 0.25) (layer F.Cu) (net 6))
 (segment (start 62.8 37.9753) (end 58.7553 42.02) (width 0.25) (layer F.Cu) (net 6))
 (segment (start 58.7553 42.02) (end 45.01 42.02) (width 0.25) (layer F.Cu) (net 6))
 (segment (start 47.55 40.75) (end 48.6353 40.75) (width 0.25) (layer B.Cu) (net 7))
 (segment (start 87.3 51.5) (end 85.05 49.25) (width 0.25) (layer B.Cu) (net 7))
 (segment (start 85.05 49.25) (end 57.1353 49.25) (width 0.25) (layer B.Cu) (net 7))
 (segment (start 57.1353 49.25) (end 48.6353 40.75) (width 0.25) (layer B.Cu) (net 7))
 (segment (start 66.8 51.6) (end 66.8 53.1753) (width 0.25) (layer F.Cu) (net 7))
 (segment (start 66.8 53.1753) (end 67.2893 53.6646) (width 0.25) (layer F.Cu) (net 7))
 (segment (start 67.2893 53.6646) (end 85.1354 53.6646) (width 0.25) (layer F.Cu) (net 7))
 (segment (start 85.1354 53.6646) (end 87.3 51.5) (width 0.25) (layer F.Cu) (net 7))
 (segment (start 70.8 36.4) (end 70.8 37.9753) (width 0.25) (layer F.Cu) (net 8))
 (segment (start 70.8 37.9753) (end 72.8517 40.027) (width 0.25) (layer F.Cu) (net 8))
 (segment (start 72.8517 40.027) (end 75.2547 40.027) (width 0.25) (layer F.Cu) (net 8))
 (segment (start 75.2547 40.027) (end 77.3 42.0723) (width 0.25) (layer F.Cu) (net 8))
 (segment (start 77.3 42.0723) (end 77.3 42.75) (width 0.25) (layer F.Cu) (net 8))
 (segment (start 64.8 36.4) (end 64.8 34.8247) (width 0.25) (layer F.Cu) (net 10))
 (segment (start 64.8 34.8247) (end 73.4747 34.8247) (width 0.25) (layer F.Cu) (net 10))
 (segment (start 73.4747 34.8247) (end 73.9082 35.2582) (width 0.25) (layer F.Cu) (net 10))
 (segment (start 73.9082 35.2582) (end 73.9082 35.8951) (width 0.25) (layer F.Cu) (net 10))
 (segment (start 73.9082 35.8951) (end 76.4484 38.4353) (width 0.25) (layer F.Cu) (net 10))
 (segment (start 76.4484 38.4353) (end 80.3328 38.4353) (width 0.25) (layer F.Cu) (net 10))
 (segment (start 80.3328 38.4353) (end 81.1475 39.25) (width 0.25) (layer F.Cu) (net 10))
 (segment (start 70.8 51.6) (end 70.8 53.1753) (width 0.25) (layer F.Cu) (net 11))
 (segment (start 70.8 53.1753) (end 75.6247 53.1753) (width 0.25) (layer F.Cu) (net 11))
 (segment (start 75.6247 53.1753) (end 77.3 51.5) (width 0.25) (layer F.Cu) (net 11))
 (segment (start 83.8 51.5) (end 77.3 51.5) (width 0.25) (layer F.Cu) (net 11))
 (segment (start 58.8 51.6) (end 58.8 53.1753) (width 0.25) (layer F.Cu) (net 12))
 (segment (start 64.8 51.6) (end 64.8 53.1753) (width 0.25) (layer F.Cu) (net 12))
 (segment (start 64.8 53.1753) (end 58.8 53.1753) (width 0.25) (layer F.Cu) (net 12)))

